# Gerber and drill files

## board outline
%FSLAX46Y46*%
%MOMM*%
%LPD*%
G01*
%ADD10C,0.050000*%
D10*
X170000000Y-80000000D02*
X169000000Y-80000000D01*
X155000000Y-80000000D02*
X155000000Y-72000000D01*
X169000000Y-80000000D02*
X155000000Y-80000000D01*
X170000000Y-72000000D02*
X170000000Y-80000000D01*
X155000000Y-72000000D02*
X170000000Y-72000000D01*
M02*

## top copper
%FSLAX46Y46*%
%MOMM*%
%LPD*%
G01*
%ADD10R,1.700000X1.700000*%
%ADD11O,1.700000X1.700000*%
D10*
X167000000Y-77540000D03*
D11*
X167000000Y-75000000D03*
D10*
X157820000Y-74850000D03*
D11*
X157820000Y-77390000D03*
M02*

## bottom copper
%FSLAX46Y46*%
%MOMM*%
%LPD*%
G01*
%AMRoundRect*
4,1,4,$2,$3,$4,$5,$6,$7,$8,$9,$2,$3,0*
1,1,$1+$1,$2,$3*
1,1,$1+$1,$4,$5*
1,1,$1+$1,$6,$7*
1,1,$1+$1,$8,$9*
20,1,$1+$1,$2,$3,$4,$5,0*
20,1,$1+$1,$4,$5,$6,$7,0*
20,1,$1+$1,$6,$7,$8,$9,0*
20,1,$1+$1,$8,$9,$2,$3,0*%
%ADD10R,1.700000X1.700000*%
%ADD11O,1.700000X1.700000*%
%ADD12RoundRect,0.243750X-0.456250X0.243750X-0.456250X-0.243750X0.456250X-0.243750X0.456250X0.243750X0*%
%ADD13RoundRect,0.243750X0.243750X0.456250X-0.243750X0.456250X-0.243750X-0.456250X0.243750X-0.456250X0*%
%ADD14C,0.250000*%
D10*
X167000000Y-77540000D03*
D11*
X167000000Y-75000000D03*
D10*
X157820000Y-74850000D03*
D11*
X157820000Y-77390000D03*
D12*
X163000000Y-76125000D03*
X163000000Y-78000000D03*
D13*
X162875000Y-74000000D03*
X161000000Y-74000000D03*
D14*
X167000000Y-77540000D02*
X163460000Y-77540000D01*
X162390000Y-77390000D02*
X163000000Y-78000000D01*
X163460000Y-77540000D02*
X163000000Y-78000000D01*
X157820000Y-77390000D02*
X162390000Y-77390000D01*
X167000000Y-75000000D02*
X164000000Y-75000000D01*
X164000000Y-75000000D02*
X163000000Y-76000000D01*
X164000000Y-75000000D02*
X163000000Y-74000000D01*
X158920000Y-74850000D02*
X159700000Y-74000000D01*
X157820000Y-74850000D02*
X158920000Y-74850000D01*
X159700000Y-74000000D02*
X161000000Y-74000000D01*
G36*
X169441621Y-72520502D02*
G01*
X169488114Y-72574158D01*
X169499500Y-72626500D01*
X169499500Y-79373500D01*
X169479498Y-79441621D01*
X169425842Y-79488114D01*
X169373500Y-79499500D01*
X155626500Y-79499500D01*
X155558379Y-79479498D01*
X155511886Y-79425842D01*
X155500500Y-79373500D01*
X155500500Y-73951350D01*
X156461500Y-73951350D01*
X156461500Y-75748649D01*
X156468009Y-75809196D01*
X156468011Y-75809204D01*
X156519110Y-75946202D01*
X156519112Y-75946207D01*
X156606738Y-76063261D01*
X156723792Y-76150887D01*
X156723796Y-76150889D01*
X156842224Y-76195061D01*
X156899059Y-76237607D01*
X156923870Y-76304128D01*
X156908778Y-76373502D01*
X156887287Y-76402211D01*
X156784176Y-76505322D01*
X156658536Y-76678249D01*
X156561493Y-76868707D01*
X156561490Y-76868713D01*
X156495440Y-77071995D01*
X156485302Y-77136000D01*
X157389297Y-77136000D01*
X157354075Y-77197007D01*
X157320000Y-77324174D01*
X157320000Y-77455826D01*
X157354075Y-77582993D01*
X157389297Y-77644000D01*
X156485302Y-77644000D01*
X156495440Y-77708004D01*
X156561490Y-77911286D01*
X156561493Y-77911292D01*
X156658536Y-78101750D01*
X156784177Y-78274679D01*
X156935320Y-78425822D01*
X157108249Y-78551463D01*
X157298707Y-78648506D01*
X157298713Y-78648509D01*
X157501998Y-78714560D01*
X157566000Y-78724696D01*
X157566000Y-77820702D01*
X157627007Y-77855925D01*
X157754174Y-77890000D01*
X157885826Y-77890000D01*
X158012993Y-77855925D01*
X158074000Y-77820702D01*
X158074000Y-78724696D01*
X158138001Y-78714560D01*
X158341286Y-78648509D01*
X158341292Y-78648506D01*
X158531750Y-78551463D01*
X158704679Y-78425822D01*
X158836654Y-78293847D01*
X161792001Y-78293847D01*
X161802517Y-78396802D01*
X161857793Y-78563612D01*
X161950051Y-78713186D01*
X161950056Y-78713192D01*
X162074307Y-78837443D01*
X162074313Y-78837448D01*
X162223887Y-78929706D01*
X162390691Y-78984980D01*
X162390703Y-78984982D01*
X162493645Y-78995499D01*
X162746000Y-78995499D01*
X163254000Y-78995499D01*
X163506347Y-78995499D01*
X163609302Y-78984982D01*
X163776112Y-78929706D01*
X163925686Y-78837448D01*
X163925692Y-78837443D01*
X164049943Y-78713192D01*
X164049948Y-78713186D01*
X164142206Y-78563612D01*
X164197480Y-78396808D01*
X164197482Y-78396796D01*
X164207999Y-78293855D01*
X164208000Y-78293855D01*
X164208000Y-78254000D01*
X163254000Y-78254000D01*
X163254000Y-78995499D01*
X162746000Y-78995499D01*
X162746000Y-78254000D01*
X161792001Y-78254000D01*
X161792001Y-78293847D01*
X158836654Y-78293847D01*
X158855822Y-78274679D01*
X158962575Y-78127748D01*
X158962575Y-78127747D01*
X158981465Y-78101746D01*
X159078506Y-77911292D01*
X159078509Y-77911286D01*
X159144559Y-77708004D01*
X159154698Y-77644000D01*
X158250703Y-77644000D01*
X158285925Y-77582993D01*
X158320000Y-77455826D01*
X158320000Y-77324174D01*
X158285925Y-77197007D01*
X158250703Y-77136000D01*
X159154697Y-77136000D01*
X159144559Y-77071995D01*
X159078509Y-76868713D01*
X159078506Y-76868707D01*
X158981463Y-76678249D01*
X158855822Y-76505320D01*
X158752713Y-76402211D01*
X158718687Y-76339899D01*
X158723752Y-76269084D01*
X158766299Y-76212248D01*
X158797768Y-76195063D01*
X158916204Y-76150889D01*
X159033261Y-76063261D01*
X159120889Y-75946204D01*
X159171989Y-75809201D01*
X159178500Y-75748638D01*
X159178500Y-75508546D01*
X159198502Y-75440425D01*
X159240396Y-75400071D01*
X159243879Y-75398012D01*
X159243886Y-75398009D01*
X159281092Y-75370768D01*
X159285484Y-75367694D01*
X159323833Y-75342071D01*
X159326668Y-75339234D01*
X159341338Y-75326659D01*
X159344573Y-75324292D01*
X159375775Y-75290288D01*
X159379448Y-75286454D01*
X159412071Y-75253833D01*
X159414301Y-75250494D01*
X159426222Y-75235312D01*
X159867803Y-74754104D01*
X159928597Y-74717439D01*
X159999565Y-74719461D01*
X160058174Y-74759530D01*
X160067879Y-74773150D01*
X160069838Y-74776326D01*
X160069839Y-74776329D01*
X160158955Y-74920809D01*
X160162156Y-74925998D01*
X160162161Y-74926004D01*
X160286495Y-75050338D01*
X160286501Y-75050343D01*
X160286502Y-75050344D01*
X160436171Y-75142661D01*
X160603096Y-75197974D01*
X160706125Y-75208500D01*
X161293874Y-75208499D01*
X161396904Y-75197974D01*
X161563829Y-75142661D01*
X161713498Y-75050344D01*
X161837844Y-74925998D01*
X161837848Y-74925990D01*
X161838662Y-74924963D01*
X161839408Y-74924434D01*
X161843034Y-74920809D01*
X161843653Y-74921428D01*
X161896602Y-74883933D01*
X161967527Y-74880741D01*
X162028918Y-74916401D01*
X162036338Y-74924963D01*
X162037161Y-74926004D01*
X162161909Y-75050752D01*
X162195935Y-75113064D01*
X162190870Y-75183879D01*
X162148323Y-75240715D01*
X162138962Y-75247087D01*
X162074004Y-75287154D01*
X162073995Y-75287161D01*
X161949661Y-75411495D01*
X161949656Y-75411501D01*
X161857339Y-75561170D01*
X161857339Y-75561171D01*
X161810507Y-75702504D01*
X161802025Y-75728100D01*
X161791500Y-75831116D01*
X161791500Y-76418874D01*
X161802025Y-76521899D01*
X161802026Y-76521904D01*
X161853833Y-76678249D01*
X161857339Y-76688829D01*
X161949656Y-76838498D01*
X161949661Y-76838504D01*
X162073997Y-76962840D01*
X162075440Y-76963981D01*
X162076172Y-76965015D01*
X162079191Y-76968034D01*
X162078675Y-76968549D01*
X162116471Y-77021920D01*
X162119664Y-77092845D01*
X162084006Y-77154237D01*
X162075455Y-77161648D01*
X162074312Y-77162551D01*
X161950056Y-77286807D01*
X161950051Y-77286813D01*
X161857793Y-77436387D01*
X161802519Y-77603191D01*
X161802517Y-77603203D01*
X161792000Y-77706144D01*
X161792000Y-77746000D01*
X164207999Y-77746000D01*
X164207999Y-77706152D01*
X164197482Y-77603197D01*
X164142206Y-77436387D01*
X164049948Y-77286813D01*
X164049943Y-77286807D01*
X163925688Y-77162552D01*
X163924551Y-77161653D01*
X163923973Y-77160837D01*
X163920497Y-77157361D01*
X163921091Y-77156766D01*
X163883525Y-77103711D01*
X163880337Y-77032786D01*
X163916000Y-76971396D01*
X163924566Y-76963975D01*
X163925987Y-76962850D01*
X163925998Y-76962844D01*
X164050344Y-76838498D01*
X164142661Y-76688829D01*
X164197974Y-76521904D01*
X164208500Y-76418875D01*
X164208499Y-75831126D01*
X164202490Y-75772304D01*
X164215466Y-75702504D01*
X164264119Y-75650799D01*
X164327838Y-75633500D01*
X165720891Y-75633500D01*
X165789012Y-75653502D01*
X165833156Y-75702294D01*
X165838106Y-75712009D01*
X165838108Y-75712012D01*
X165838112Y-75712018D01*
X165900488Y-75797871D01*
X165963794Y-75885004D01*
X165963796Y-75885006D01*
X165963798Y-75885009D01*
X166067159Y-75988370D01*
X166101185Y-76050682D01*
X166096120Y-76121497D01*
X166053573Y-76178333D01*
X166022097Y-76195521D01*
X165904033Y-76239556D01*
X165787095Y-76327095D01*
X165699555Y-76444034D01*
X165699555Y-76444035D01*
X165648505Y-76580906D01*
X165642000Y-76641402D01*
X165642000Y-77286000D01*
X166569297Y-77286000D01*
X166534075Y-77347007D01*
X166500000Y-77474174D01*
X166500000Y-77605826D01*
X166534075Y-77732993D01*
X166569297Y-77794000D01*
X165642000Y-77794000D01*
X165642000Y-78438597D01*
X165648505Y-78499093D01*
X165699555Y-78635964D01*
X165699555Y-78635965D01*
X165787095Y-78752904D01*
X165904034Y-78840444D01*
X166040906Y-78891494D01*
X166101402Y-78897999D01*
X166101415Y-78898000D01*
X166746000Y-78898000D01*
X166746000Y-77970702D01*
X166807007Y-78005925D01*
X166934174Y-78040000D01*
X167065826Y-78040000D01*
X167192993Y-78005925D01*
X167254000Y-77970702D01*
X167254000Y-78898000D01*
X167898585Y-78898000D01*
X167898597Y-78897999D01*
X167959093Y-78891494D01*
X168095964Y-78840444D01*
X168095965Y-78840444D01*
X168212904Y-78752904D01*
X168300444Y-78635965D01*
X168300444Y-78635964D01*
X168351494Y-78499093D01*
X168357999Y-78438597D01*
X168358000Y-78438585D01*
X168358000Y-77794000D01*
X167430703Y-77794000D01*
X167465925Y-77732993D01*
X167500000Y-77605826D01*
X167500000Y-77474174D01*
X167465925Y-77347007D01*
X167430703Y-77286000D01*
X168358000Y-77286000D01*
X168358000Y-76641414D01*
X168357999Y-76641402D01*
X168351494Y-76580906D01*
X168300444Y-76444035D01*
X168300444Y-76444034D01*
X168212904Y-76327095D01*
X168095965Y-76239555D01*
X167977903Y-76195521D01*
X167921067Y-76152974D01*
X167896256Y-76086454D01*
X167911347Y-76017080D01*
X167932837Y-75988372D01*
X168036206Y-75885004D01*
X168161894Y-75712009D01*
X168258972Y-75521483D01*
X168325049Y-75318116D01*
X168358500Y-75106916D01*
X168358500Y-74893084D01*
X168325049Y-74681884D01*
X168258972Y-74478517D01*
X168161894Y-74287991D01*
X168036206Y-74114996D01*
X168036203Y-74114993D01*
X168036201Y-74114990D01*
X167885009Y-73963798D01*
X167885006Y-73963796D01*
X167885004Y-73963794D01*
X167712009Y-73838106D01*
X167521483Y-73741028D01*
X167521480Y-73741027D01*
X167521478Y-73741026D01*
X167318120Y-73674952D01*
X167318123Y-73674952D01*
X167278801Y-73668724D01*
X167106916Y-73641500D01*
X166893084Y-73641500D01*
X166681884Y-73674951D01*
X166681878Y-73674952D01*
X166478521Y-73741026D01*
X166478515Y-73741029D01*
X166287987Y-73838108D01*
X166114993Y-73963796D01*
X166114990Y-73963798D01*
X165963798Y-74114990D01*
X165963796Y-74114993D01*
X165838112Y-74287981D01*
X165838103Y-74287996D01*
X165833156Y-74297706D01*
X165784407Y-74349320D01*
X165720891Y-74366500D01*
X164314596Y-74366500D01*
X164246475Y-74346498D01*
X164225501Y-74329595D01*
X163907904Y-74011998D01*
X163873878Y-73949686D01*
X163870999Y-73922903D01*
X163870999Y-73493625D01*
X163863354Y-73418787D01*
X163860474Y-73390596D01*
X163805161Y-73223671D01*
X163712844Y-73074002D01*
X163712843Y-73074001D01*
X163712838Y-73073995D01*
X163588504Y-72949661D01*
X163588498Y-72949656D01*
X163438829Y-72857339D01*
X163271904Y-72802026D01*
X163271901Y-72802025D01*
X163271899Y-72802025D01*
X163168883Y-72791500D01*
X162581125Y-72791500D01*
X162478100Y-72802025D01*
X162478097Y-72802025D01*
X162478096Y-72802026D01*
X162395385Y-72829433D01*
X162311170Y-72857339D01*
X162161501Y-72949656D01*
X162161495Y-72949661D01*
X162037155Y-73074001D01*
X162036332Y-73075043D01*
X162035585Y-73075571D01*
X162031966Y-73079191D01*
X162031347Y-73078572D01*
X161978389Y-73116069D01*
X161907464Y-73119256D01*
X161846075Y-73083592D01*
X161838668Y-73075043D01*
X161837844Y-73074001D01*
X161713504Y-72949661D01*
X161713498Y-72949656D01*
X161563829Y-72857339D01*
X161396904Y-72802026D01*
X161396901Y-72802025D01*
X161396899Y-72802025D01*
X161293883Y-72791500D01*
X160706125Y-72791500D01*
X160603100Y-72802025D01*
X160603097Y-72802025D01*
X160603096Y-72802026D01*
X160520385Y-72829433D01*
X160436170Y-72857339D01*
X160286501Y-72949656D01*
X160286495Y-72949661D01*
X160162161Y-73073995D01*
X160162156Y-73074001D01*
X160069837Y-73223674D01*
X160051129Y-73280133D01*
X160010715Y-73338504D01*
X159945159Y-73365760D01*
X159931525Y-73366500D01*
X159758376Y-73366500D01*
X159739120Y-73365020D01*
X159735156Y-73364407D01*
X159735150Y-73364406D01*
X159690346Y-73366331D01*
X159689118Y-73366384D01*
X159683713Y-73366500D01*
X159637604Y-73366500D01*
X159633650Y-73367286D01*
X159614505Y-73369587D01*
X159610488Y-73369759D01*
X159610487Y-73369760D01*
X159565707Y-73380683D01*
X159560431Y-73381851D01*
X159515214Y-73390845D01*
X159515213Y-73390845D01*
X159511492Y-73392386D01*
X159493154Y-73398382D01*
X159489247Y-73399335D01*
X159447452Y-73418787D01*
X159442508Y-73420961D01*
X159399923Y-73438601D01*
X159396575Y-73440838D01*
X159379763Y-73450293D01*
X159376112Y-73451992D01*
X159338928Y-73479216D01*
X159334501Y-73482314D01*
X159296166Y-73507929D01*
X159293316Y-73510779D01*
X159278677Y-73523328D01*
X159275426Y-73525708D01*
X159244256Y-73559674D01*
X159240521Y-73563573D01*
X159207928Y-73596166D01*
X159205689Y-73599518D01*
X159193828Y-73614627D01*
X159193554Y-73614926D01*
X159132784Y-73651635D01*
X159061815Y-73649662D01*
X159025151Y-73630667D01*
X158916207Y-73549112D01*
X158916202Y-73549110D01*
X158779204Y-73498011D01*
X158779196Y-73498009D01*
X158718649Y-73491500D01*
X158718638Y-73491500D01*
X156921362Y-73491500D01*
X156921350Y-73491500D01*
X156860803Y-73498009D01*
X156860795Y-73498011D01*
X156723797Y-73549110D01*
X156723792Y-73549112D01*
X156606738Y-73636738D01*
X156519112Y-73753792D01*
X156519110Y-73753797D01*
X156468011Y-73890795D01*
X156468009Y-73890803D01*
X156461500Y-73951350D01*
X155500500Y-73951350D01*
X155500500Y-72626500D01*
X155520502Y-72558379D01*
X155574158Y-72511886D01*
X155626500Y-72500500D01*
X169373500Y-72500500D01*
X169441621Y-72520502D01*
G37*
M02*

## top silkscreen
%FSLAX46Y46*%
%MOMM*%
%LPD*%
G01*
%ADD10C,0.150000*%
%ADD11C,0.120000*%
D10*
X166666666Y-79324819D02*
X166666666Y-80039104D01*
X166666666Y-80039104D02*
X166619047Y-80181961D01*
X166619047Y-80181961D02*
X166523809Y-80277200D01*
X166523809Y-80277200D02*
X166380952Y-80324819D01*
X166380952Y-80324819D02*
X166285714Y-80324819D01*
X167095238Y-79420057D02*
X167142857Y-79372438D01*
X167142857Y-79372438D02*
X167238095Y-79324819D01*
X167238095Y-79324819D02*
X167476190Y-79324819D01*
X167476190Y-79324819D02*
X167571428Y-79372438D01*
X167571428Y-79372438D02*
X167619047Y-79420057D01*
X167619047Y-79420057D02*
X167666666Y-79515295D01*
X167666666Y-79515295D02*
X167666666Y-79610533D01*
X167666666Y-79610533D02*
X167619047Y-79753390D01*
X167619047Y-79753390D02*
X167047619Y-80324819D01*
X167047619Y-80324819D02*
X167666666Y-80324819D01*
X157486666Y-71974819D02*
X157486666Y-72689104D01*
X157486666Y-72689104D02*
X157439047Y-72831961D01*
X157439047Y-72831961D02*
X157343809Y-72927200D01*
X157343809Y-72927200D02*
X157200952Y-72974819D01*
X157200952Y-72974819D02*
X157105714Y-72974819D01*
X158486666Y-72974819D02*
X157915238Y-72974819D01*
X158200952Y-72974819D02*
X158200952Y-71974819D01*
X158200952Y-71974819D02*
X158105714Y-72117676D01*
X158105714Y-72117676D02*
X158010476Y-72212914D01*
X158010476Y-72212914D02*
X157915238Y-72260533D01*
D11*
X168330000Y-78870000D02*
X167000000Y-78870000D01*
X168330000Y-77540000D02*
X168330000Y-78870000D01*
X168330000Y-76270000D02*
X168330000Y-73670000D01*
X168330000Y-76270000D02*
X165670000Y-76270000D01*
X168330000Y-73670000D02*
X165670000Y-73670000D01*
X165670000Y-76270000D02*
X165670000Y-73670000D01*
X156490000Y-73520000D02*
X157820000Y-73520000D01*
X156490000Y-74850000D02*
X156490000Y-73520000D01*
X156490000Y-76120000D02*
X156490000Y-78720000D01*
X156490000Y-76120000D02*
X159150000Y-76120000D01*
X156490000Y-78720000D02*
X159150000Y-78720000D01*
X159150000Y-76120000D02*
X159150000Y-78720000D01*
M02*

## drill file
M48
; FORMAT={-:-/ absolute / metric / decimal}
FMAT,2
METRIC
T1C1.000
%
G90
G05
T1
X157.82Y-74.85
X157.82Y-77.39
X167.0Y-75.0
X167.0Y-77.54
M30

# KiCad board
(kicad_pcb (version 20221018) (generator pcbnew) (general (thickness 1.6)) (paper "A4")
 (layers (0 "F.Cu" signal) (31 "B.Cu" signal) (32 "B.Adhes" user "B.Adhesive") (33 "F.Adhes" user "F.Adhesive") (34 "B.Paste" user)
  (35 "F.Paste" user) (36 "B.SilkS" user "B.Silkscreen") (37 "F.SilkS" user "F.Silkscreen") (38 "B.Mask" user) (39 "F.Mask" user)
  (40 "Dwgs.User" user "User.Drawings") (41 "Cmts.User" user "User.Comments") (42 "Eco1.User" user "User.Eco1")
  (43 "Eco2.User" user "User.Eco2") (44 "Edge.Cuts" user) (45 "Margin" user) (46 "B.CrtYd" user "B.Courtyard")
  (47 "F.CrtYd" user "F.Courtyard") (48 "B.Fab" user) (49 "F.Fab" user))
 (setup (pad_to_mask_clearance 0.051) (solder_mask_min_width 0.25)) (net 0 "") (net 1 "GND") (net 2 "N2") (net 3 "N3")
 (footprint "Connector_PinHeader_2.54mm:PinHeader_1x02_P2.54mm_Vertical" (layer "F.Cu") (at 167 77.54 180)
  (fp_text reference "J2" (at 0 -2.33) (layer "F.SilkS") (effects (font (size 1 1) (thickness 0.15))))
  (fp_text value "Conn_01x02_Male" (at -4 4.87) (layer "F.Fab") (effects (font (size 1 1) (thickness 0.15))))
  (fp_line (start -1.33 -1.33) (end 0 -1.33) (stroke (width 0.12) (type solid)) (layer "F.SilkS"))
  (fp_line (start -1.33 0) (end -1.33 -1.33) (stroke (width 0.12) (type solid)) (layer "F.SilkS"))
  (fp_line (start -1.33 1.27) (end -1.33 3.87) (stroke (width 0.12) (type solid)) (layer "F.SilkS"))
  (fp_line (start -1.33 1.27) (end 1.33 1.27) (stroke (width 0.12) (type solid)) (layer "F.SilkS"))
  (fp_line (start -1.33 3.87) (end 1.33 3.87) (stroke (width 0.12) (type solid)) (layer "F.SilkS"))
  (fp_line (start 1.33 1.27) (end 1.33 3.87) (stroke (width 0.12) (type solid)) (layer "F.SilkS"))
  (pad "1" thru_hole rect (at 0 0 180) (size 1.7 1.7) (drill 1) (layers "*.Cu" "*.Mask") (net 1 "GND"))
  (pad "2" thru_hole oval (at 0 2.54 180) (size 1.7 1.7) (drill 1) (layers "*.Cu" "*.Mask") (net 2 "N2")))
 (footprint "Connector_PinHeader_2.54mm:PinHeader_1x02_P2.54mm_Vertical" (layer "F.Cu") (at 157.82 74.85)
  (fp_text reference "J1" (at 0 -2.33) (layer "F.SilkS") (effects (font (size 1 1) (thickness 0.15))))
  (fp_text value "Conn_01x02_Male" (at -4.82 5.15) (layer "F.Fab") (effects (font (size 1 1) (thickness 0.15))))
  (fp_line (start -1.33 -1.33) (end 0 -1.33) (stroke (width 0.12) (type solid)) (layer "F.SilkS"))
  (fp_line (start -1.33 0) (end -1.33 -1.33) (stroke (width 0.12) (type solid)) (layer "F.SilkS"))
  (fp_line (start -1.33 1.27) (end -1.33 3.87) (stroke (width 0.12) (type solid)) (layer "F.SilkS"))
  (fp_line (start -1.33 1.27) (end 1.33 1.27) (stroke (width 0.12) (type solid)) (layer "F.SilkS"))
  (fp_line (start -1.33 3.87) (end 1.33 3.87) (stroke (width 0.12) (type solid)) (layer "F.SilkS"))
  (fp_line (start 1.33 1.27) (end 1.33 3.87) (stroke (width 0.12) (type solid)) (layer "F.SilkS"))
  (pad "1" thru_hole rect (at 0 0) (size 1.7 1.7) (drill 1) (layers "*.Cu" "*.Mask") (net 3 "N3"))
  (pad "2" thru_hole oval (at 0 2.54) (size 1.7 1.7) (drill 1) (layers "*.Cu" "*.Mask") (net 1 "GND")))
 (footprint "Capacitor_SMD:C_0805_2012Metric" (layer "B.Cu") (at 163 77.0625 -90)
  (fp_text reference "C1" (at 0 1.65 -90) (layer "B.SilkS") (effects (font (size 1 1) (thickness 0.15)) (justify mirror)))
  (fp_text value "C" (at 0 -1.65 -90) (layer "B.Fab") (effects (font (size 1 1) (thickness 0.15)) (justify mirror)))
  (pad "1" smd roundrect (at -0.9375 0 270) (size 0.975 1.4) (layers "B.Cu" "B.Paste" "B.Mask") (roundrect_rratio 0.25) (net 2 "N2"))
  (pad "2" smd roundrect (at 0.9375 0 270) (size 0.975 1.4) (layers "B.Cu" "B.Paste" "B.Mask") (roundrect_rratio 0.25) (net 1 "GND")))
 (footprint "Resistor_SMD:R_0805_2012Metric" (layer "B.Cu") (at 161.9375 74 180)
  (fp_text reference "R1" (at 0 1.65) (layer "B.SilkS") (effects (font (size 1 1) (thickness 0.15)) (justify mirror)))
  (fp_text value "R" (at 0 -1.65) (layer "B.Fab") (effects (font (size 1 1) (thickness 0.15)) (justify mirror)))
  (pad "1" smd roundrect (at -0.9375 0 180) (size 0.975 1.4) (layers "B.Cu" "B.Paste" "B.Mask") (roundrect_rratio 0.25) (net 2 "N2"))
  (pad "2" smd roundrect (at 0.9375 0 180) (size 0.975 1.4) (layers "B.Cu" "B.Paste" "B.Mask") (roundrect_rratio 0.25) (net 3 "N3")))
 (gr_line (start 170 80) (end 169 80) (stroke (width 0.05) (type solid)) (layer "Edge.Cuts"))
 (gr_line (start 155 80) (end 155 72) (stroke (width 0.05) (type solid)) (layer "Edge.Cuts"))
 (gr_line (start 169 80) (end 155 80) (stroke (width 0.05) (type solid)) (layer "Edge.Cuts"))
 (gr_line (start 170 72) (end 170 80) (stroke (width 0.05) (type solid)) (layer "Edge.Cuts"))
 (gr_line (start 155 72) (end 170 72) (stroke (width 0.05) (type solid)) (layer "Edge.Cuts"))
 (segment (start 167 77.54) (end 163.46 77.54) (width 0.25) (layer "B.Cu") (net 1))
 (segment (start 162.39 77.39) (end 163 78) (width 0.25) (layer "B.Cu") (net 1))
 (segment (start 163.46 77.54) (end 163 78) (width 0.25) (layer "B.Cu") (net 1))
 (segment (start 157.82 77.39) (end 162.39 77.39) (width 0.25) (layer "B.Cu") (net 1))
 (segment (start 167 75) (end 164 75) (width 0.25) (layer "B.Cu") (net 2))
 (segment (start 164 75) (end 163 76) (width 0.25) (layer "B.Cu") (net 2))
 (segment (start 164 75) (end 163 74) (width 0.25) (layer "B.Cu") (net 2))
 (segment (start 158.92 74.85) (end 159.7 74) (width 0.25) (layer "B.Cu") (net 3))
 (segment (start 157.82 74.85) (end 158.92 74.85) (width 0.25) (layer "B.Cu") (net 3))
 (segment (start 159.7 74) (end 161 74) (width 0.25) (layer "B.Cu") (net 3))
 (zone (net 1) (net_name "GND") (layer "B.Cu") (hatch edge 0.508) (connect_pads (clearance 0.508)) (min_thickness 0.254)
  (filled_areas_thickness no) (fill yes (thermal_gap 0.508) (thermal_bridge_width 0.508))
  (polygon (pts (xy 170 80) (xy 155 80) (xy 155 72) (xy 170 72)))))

